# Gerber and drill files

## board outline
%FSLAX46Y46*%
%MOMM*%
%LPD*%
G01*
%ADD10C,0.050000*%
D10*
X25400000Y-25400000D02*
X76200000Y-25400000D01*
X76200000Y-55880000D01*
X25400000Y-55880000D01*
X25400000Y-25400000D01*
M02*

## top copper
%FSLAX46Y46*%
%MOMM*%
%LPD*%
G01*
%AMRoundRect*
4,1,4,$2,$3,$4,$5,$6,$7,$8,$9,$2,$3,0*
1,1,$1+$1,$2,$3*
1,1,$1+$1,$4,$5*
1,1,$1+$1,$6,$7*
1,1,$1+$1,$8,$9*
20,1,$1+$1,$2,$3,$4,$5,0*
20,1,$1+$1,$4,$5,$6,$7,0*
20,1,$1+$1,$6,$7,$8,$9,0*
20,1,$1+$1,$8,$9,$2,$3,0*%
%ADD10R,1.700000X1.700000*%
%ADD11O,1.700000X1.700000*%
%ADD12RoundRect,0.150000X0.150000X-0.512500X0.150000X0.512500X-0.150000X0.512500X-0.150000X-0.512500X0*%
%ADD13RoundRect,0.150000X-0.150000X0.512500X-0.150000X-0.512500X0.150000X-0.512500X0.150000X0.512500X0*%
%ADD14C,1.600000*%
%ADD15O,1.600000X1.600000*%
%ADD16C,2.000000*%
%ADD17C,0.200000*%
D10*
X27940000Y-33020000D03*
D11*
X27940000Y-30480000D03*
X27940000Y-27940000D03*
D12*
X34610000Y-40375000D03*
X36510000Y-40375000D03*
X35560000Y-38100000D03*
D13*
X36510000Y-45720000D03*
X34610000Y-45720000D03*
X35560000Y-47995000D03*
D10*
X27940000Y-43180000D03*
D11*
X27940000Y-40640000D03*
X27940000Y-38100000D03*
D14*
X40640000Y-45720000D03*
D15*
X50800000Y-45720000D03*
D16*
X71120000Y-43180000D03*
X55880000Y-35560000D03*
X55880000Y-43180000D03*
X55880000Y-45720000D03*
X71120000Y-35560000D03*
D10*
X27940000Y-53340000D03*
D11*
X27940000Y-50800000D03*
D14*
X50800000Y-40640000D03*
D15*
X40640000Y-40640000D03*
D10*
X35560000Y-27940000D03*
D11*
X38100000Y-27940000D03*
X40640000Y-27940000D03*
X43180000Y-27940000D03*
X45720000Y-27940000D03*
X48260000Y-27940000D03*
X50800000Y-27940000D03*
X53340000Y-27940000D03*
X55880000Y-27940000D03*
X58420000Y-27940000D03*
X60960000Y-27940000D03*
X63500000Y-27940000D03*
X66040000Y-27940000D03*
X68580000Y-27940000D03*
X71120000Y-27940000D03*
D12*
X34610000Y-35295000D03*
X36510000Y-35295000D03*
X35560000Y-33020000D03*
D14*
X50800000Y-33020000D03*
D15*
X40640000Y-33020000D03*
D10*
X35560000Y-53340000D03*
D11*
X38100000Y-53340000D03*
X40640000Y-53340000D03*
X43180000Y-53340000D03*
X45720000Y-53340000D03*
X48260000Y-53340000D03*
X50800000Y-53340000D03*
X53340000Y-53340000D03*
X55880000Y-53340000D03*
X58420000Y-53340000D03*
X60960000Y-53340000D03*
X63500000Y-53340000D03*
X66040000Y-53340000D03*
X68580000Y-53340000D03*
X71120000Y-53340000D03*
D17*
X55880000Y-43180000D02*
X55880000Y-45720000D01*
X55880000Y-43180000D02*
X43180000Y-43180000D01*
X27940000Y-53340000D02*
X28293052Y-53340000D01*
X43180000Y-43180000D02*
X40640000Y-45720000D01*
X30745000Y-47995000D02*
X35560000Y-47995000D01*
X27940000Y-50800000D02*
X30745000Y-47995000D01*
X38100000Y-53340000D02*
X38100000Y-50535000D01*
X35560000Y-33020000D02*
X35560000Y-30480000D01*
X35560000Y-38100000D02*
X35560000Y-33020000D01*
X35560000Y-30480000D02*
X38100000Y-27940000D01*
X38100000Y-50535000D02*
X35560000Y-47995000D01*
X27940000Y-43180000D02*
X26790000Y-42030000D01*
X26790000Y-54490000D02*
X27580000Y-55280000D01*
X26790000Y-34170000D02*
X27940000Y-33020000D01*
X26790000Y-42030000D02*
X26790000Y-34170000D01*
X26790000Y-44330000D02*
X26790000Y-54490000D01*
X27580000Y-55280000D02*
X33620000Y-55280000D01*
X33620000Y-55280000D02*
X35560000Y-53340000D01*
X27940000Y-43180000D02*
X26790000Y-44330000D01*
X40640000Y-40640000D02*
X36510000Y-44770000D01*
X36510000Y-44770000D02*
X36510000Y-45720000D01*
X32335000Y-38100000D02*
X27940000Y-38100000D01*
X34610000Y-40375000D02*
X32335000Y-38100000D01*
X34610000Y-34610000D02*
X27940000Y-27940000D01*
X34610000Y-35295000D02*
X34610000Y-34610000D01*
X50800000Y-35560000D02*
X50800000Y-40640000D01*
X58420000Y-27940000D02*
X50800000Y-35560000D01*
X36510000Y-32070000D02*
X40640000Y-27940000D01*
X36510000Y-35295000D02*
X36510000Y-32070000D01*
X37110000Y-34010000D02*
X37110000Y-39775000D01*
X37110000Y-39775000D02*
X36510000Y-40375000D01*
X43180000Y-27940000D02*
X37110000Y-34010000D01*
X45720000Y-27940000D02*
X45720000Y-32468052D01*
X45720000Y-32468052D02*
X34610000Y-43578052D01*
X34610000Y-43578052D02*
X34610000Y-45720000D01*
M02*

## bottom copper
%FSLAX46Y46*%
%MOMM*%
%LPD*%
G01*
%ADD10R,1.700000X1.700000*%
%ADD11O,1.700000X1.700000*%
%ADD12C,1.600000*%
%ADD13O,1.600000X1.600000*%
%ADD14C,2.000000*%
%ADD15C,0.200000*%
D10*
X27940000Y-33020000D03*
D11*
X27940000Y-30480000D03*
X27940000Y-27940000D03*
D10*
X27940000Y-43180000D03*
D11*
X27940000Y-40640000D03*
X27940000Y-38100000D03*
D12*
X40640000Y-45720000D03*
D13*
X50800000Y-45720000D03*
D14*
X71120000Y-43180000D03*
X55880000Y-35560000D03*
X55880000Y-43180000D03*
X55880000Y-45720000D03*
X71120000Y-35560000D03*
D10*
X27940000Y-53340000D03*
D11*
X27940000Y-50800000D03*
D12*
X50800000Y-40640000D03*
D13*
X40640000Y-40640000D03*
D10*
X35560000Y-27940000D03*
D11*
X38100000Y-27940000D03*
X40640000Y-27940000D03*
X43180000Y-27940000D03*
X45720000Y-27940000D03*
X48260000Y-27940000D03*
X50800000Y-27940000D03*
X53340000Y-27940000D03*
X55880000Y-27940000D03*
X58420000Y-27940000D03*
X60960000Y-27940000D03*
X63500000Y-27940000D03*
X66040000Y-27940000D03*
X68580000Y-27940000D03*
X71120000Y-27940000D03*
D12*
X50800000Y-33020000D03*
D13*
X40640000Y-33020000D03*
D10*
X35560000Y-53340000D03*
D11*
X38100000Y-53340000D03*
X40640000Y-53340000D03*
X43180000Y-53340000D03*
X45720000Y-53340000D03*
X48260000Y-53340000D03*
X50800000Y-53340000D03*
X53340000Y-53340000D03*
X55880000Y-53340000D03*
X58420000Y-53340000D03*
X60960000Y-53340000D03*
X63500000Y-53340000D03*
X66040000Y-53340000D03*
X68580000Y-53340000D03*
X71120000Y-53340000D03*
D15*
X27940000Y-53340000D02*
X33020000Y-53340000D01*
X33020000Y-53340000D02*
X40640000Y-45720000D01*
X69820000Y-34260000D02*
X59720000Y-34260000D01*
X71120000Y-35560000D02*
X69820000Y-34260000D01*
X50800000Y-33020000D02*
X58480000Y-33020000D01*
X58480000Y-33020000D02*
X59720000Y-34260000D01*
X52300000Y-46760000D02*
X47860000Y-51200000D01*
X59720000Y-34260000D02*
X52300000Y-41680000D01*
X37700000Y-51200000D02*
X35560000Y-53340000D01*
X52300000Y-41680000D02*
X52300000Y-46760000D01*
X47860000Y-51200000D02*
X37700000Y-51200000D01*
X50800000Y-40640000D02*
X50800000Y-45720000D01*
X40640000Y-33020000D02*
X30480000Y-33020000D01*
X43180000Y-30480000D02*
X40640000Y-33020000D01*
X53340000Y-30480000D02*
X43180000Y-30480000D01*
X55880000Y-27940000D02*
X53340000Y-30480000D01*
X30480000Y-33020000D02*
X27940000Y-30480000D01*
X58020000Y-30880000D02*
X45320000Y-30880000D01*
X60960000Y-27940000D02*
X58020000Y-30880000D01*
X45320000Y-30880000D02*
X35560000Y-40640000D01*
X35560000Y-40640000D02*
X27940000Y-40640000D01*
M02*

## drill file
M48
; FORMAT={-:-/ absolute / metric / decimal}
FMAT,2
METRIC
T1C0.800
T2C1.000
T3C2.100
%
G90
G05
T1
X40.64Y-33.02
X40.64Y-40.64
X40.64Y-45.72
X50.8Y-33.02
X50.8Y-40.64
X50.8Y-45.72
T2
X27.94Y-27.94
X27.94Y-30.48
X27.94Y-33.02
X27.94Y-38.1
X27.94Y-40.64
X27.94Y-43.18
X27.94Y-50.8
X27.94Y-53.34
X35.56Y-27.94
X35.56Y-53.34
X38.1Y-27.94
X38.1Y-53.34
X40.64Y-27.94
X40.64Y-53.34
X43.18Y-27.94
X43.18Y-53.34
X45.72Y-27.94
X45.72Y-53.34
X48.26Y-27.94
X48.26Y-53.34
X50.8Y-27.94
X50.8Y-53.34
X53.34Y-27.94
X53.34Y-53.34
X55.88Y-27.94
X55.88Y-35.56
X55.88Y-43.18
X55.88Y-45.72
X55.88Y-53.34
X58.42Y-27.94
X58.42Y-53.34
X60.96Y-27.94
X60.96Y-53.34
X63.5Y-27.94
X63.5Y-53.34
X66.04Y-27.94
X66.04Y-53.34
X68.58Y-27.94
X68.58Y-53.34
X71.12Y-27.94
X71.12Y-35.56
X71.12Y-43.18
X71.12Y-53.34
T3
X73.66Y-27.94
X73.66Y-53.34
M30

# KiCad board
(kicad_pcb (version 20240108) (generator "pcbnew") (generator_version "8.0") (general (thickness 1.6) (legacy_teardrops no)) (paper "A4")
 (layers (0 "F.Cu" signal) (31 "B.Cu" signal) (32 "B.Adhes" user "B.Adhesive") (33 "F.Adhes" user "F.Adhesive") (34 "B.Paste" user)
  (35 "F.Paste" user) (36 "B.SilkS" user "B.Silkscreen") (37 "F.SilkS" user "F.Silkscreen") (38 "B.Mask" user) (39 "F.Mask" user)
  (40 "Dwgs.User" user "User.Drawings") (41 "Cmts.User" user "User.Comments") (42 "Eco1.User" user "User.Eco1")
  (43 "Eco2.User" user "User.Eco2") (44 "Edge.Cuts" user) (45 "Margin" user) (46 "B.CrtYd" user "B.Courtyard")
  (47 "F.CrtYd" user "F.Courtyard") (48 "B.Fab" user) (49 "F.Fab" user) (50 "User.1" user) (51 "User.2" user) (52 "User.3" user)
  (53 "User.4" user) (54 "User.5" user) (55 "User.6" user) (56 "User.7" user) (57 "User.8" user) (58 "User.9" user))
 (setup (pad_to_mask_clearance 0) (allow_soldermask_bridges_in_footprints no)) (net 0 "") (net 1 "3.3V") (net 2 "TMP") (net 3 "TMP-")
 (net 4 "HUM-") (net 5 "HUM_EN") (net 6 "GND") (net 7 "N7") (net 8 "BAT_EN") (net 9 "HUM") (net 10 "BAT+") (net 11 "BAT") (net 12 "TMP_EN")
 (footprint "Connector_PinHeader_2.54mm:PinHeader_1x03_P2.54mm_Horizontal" (layer "F.Cu") (at 27.94 33.02 180)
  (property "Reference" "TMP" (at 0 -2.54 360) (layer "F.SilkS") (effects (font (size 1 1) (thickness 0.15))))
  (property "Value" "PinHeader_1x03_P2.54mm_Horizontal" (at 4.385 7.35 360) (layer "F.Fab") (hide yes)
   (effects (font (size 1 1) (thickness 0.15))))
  (pad "1" thru_hole rect (at 0 0 180) (size 1.7 1.7) (drill 1) (layers "*.Cu" "*.Mask") (remove_unused_layers no) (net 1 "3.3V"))
  (pad "2" thru_hole oval (at 0 2.54 180) (size 1.7 1.7) (drill 1) (layers "*.Cu" "*.Mask") (remove_unused_layers no) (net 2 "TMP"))
  (pad "3" thru_hole oval (at 0 5.08 180) (size 1.7 1.7) (drill 1) (layers "*.Cu" "*.Mask") (remove_unused_layers no) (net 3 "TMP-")))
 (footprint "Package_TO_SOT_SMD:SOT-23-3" (layer "F.Cu") (at 35.56 39.2375 90)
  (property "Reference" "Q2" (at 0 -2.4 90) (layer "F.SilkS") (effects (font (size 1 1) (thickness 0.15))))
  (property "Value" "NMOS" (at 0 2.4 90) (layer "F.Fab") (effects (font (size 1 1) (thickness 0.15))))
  (pad "1" smd roundrect (at -1.1375 -0.95 90) (size 1.325 0.6) (layers "F.Cu" "F.Paste" "F.Mask") (roundrect_rratio 0.25) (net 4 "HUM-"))
  (pad "2" smd roundrect (at -1.1375 0.95 90) (size 1.325 0.6) (layers "F.Cu" "F.Paste" "F.Mask") (roundrect_rratio 0.25) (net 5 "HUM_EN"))
  (pad "3" smd roundrect (at 1.1375 0 90) (size 1.325 0.6) (layers "F.Cu" "F.Paste" "F.Mask") (roundrect_rratio 0.25) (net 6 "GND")))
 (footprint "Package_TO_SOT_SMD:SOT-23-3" (layer "F.Cu") (at 35.56 46.8575 -90)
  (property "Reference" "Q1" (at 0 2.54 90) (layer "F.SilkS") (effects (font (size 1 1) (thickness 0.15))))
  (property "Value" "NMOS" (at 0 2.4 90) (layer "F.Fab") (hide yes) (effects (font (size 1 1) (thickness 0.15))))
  (pad "1" smd roundrect (at -1.1375 -0.95 270) (size 1.325 0.6) (layers "F.Cu" "F.Paste" "F.Mask") (roundrect_rratio 0.25) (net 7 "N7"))
  (pad "2" smd roundrect (at -1.1375 0.95 270) (size 1.325 0.6) (layers "F.Cu" "F.Paste" "F.Mask") (roundrect_rratio 0.25) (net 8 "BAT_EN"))
  (pad "3" smd roundrect (at 1.1375 0 270) (size 1.325 0.6) (layers "F.Cu" "F.Paste" "F.Mask") (roundrect_rratio 0.25) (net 6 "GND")))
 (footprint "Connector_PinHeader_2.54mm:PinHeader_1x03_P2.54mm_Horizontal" (layer "F.Cu") (at 27.94 43.18 180)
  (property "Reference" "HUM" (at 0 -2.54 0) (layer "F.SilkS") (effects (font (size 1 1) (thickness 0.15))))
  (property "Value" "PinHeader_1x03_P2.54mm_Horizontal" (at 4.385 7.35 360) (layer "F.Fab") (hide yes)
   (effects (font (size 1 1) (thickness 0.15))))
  (pad "1" thru_hole rect (at 0 0 180) (size 1.7 1.7) (drill 1) (layers "*.Cu" "*.Mask") (remove_unused_layers no) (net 1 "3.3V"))
  (pad "2" thru_hole oval (at 0 2.54 180) (size 1.7 1.7) (drill 1) (layers "*.Cu" "*.Mask") (remove_unused_layers no) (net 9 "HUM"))
  (pad "3" thru_hole oval (at 0 5.08 180) (size 1.7 1.7) (drill 1) (layers "*.Cu" "*.Mask") (remove_unused_layers no) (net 4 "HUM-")))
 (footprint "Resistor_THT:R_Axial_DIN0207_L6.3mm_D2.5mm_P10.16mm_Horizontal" (layer "F.Cu") (at 40.64 45.72)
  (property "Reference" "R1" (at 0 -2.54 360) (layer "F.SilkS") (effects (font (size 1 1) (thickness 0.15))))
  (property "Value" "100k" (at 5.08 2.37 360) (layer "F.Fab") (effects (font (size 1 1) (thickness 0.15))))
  (pad "1" thru_hole circle (at 0 0) (size 1.6 1.6) (drill 0.8) (layers "*.Cu" "*.Mask") (remove_unused_layers no) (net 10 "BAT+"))
  (pad "2" thru_hole oval (at 10.16 0) (size 1.6 1.6) (drill 0.8) (layers "*.Cu" "*.Mask") (remove_unused_layers no) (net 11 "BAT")))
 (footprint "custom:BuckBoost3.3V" (layer "F.Cu") (at 63.5 40.64 90)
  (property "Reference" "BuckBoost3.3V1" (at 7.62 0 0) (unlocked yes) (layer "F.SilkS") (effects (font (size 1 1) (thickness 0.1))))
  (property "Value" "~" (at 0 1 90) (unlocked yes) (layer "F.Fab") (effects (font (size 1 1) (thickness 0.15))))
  (pad "1" thru_hole circle (at -2.54 7.62 90) (size 2 2) (drill 1) (layers "*.Cu" "*.Mask") (remove_unused_layers no) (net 6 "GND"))
  (pad "1" thru_hole circle (at 5.08 -7.62 90) (size 2 2) (drill 1) (layers "*.Cu" "*.Mask") (remove_unused_layers no) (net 6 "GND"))
  (pad "2" thru_hole circle (at -2.54 -7.62 90) (size 2 2) (drill 1) (layers "*.Cu" "*.Mask") (remove_unused_layers no) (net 10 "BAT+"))
  (pad "3" thru_hole circle (at -5.08 -7.62 90) (size 2 2) (drill 1) (layers "*.Cu" "*.Mask") (remove_unused_layers no) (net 10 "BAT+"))
  (pad "4" thru_hole circle (at 5.08 7.62 90) (size 2 2) (drill 1) (layers "*.Cu" "*.Mask") (remove_unused_layers no) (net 1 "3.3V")))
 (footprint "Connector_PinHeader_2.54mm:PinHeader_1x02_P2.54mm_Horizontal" (layer "F.Cu") (at 27.94 53.34 180)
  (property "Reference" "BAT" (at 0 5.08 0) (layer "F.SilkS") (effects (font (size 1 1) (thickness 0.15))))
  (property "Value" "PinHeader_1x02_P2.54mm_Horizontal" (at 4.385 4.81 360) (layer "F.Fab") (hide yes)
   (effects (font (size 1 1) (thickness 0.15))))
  (pad "1" thru_hole rect (at 0 0 180) (size 1.7 1.7) (drill 1) (layers "*.Cu" "*.Mask") (remove_unused_layers no) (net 10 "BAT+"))
  (pad "2" thru_hole oval (at 0 2.54 180) (size 1.7 1.7) (drill 1) (layers "*.Cu" "*.Mask") (remove_unused_layers no) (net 6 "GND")))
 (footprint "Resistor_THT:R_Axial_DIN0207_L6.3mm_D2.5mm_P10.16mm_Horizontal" (layer "F.Cu") (at 50.8 40.64 180)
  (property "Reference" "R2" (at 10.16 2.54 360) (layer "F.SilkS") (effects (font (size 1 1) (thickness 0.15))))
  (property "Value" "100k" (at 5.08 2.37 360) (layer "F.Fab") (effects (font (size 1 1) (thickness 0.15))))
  (pad "1" thru_hole circle (at 0 0 180) (size 1.6 1.6) (drill 0.8) (layers "*.Cu" "*.Mask") (remove_unused_layers no) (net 11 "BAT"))
  (pad "2" thru_hole oval (at 10.16 0 180) (size 1.6 1.6) (drill 0.8) (layers "*.Cu" "*.Mask") (remove_unused_layers no) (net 7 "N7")))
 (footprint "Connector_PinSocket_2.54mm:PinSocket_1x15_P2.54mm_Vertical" (layer "F.Cu") (at 35.56 27.94 90)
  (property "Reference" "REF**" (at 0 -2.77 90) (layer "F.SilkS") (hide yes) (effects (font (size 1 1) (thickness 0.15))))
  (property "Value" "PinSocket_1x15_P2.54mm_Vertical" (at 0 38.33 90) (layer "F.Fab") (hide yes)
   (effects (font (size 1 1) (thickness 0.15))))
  (pad "1" thru_hole rect (at 0 0 90) (size 1.7 1.7) (drill 1) (layers "*.Cu" "*.Mask") (remove_unused_layers no))
  (pad "2" thru_hole oval (at 0 2.54 90) (size 1.7 1.7) (drill 1) (layers "*.Cu" "*.Mask") (remove_unused_layers no) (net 6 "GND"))
  (pad "3" thru_hole oval (at 0 5.08 90) (size 1.7 1.7) (drill 1) (layers "*.Cu" "*.Mask") (remove_unused_layers no) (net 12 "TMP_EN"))
  (pad "4" thru_hole oval (at 0 7.62 90) (size 1.7 1.7) (drill 1) (layers "*.Cu" "*.Mask") (remove_unused_layers no) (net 5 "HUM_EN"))
  (pad "5" thru_hole oval (at 0 10.16 90) (size 1.7 1.7) (drill 1) (layers "*.Cu" "*.Mask") (remove_unused_layers no) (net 8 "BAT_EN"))
  (pad "6" thru_hole oval (at 0 12.7 90) (size 1.7 1.7) (drill 1) (layers "*.Cu" "*.Mask") (remove_unused_layers no))
  (pad "7" thru_hole oval (at 0 15.24 90) (size 1.7 1.7) (drill 1) (layers "*.Cu" "*.Mask") (remove_unused_layers no))
  (pad "8" thru_hole oval (at 0 17.78 90) (size 1.7 1.7) (drill 1) (layers "*.Cu" "*.Mask") (remove_unused_layers no))
  (pad "9" thru_hole oval (at 0 20.32 90) (size 1.7 1.7) (drill 1) (layers "*.Cu" "*.Mask") (remove_unused_layers no) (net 2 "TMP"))
  (pad "10" thru_hole oval (at 0 22.86 90) (size 1.7 1.7) (drill 1) (layers "*.Cu" "*.Mask") (remove_unused_layers no) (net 11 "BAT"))
  (pad "11" thru_hole oval (at 0 25.4 90) (size 1.7 1.7) (drill 1) (layers "*.Cu" "*.Mask") (remove_unused_layers no) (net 9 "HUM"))
  (pad "12" thru_hole oval (at 0 27.94 90) (size 1.7 1.7) (drill 1) (layers "*.Cu" "*.Mask") (remove_unused_layers no))
  (pad "13" thru_hole oval (at 0 30.48 90) (size 1.7 1.7) (drill 1) (layers "*.Cu" "*.Mask") (remove_unused_layers no))
  (pad "14" thru_hole oval (at 0 33.02 90) (size 1.7 1.7) (drill 1) (layers "*.Cu" "*.Mask") (remove_unused_layers no))
  (pad "15" thru_hole oval (at 0 35.56 90) (size 1.7 1.7) (drill 1) (layers "*.Cu" "*.Mask") (remove_unused_layers no)))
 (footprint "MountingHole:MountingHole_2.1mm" (layer "F.Cu") (at 73.66 53.34)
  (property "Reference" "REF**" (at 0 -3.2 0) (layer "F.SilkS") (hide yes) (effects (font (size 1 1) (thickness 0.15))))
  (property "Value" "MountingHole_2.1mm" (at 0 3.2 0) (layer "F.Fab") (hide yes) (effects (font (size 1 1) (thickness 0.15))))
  (pad "" np_thru_hole circle (at 0 0) (size 2.1 2.1) (drill 2.1) (layers "*.Cu" "*.Mask")))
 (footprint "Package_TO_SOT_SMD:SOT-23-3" (layer "F.Cu") (at 35.56 34.1575 90)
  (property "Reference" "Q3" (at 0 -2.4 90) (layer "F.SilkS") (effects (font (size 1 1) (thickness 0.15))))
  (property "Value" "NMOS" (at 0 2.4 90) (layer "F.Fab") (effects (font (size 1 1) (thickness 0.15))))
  (pad "1" smd roundrect (at -1.1375 -0.95 90) (size 1.325 0.6) (layers "F.Cu" "F.Paste" "F.Mask") (roundrect_rratio 0.25) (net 3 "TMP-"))
  (pad "2" smd roundrect (at -1.1375 0.95 90) (size 1.325 0.6) (layers "F.Cu" "F.Paste" "F.Mask") (roundrect_rratio 0.25) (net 12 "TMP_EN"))
  (pad "3" smd roundrect (at 1.1375 0 90) (size 1.325 0.6) (layers "F.Cu" "F.Paste" "F.Mask") (roundrect_rratio 0.25) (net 6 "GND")))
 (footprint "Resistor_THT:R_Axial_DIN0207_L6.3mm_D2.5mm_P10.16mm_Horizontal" (layer "F.Cu") (at 50.8 33.02 180)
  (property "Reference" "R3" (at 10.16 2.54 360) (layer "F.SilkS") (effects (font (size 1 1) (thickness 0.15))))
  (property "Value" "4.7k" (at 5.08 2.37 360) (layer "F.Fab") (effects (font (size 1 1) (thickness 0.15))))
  (pad "1" thru_hole circle (at 0 0 180) (size 1.6 1.6) (drill 0.8) (layers "*.Cu" "*.Mask") (remove_unused_layers no) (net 1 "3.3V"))
  (pad "2" thru_hole oval (at 10.16 0 180) (size 1.6 1.6) (drill 0.8) (layers "*.Cu" "*.Mask") (remove_unused_layers no) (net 2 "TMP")))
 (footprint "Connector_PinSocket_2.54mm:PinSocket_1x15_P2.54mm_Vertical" (layer "F.Cu") (at 35.56 53.34 90)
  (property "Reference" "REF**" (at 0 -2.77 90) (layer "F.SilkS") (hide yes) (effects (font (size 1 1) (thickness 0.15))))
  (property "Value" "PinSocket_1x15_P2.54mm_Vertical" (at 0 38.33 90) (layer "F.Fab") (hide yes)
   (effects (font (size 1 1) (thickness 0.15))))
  (pad "1" thru_hole rect (at 0 0 90) (size 1.7 1.7) (drill 1) (layers "*.Cu" "*.Mask") (remove_unused_layers no) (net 1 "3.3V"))
  (pad "2" thru_hole oval (at 0 2.54 90) (size 1.7 1.7) (drill 1) (layers "*.Cu" "*.Mask") (remove_unused_layers no) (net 6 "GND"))
  (pad "3" thru_hole oval (at 0 5.08 90) (size 1.7 1.7) (drill 1) (layers "*.Cu" "*.Mask") (remove_unused_layers no))
  (pad "4" thru_hole oval (at 0 7.62 90) (size 1.7 1.7) (drill 1) (layers "*.Cu" "*.Mask") (remove_unused_layers no))
  (pad "5" thru_hole oval (at 0 10.16 90) (size 1.7 1.7) (drill 1) (layers "*.Cu" "*.Mask") (remove_unused_layers no))
  (pad "6" thru_hole oval (at 0 12.7 90) (size 1.7 1.7) (drill 1) (layers "*.Cu" "*.Mask") (remove_unused_layers no))
  (pad "7" thru_hole oval (at 0 15.24 90) (size 1.7 1.7) (drill 1) (layers "*.Cu" "*.Mask") (remove_unused_layers no))
  (pad "8" thru_hole oval (at 0 17.78 90) (size 1.7 1.7) (drill 1) (layers "*.Cu" "*.Mask") (remove_unused_layers no))
  (pad "9" thru_hole oval (at 0 20.32 90) (size 1.7 1.7) (drill 1) (layers "*.Cu" "*.Mask") (remove_unused_layers no))
  (pad "10" thru_hole oval (at 0 22.86 90) (size 1.7 1.7) (drill 1) (layers "*.Cu" "*.Mask") (remove_unused_layers no))
  (pad "11" thru_hole oval (at 0 25.4 90) (size 1.7 1.7) (drill 1) (layers "*.Cu" "*.Mask") (remove_unused_layers no))
  (pad "12" thru_hole oval (at 0 27.94 90) (size 1.7 1.7) (drill 1) (layers "*.Cu" "*.Mask") (remove_unused_layers no))
  (pad "13" thru_hole oval (at 0 30.48 90) (size 1.7 1.7) (drill 1) (layers "*.Cu" "*.Mask") (remove_unused_layers no))
  (pad "14" thru_hole oval (at 0 33.02 90) (size 1.7 1.7) (drill 1) (layers "*.Cu" "*.Mask") (remove_unused_layers no))
  (pad "15" thru_hole oval (at 0 35.56 90) (size 1.7 1.7) (drill 1) (layers "*.Cu" "*.Mask") (remove_unused_layers no)))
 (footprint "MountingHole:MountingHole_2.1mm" (layer "F.Cu") (at 73.66 27.94)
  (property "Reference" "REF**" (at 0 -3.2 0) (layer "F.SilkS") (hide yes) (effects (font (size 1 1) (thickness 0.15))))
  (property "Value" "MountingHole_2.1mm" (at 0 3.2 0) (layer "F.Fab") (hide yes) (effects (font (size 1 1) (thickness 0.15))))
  (pad "" np_thru_hole circle (at 0 0) (size 2.1 2.1) (drill 2.1) (layers "*.Cu" "*.Mask")))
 (gr_rect (start 25.4 25.4) (end 76.2 55.88) (stroke (width 0.05) (type default)) (fill none) (layer "Edge.Cuts"))
 (segment (start 55.88 43.18) (end 55.88 45.72) (width 0.2) (layer "F.Cu") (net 10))
 (segment (start 55.88 43.18) (end 43.18 43.18) (width 0.2) (layer "F.Cu") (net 10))
 (segment (start 27.94 53.34) (end 28.293052 53.34) (width 0.2) (layer "F.Cu") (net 10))
 (segment (start 43.18 43.18) (end 40.64 45.72) (width 0.2) (layer "F.Cu") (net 10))
 (segment (start 27.94 53.34) (end 33.02 53.34) (width 0.2) (layer "B.Cu") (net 10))
 (segment (start 33.02 53.34) (end 40.64 45.72) (width 0.2) (layer "B.Cu") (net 10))
 (segment (start 30.745 47.995) (end 35.56 47.995) (width 0.2) (layer "F.Cu") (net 6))
 (segment (start 27.94 50.8) (end 30.745 47.995) (width 0.2) (layer "F.Cu") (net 6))
 (segment (start 38.1 53.34) (end 38.1 50.535) (width 0.2) (layer "F.Cu") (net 6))
 (segment (start 35.56 33.02) (end 35.56 30.48) (width 0.2) (layer "F.Cu") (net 6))
 (segment (start 35.56 38.1) (end 35.56 33.02) (width 0.2) (layer "F.Cu") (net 6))
 (segment (start 35.56 30.48) (end 38.1 27.94) (width 0.2) (layer "F.Cu") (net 6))
 (segment (start 38.1 50.535) (end 35.56 47.995) (width 0.2) (layer "F.Cu") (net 6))
 (segment (start 27.94 43.18) (end 26.79 42.03) (width 0.2) (layer "F.Cu") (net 1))
 (segment (start 26.79 54.49) (end 27.58 55.28) (width 0.2) (layer "F.Cu") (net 1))
 (segment (start 26.79 34.17) (end 27.94 33.02) (width 0.2) (layer "F.Cu") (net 1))
 (segment (start 26.79 42.03) (end 26.79 34.17) (width 0.2) (layer "F.Cu") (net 1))
 (segment (start 26.79 44.33) (end 26.79 54.49) (width 0.2) (layer "F.Cu") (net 1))
 (segment (start 27.58 55.28) (end 33.62 55.28) (width 0.2) (layer "F.Cu") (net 1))
 (segment (start 33.62 55.28) (end 35.56 53.34) (width 0.2) (layer "F.Cu") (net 1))
 (segment (start 27.94 43.18) (end 26.79 44.33) (width 0.2) (layer "F.Cu") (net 1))
 (segment (start 69.82 34.26) (end 59.72 34.26) (width 0.2) (layer "B.Cu") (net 1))
 (segment (start 71.12 35.56) (end 69.82 34.26) (width 0.2) (layer "B.Cu") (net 1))
 (segment (start 50.8 33.02) (end 58.48 33.02) (width 0.2) (layer "B.Cu") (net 1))
 (segment (start 58.48 33.02) (end 59.72 34.26) (width 0.2) (layer "B.Cu") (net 1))
 (segment (start 52.3 46.76) (end 47.86 51.2) (width 0.2) (layer "B.Cu") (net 1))
 (segment (start 59.72 34.26) (end 52.3 41.68) (width 0.2) (layer "B.Cu") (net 1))
 (segment (start 37.7 51.2) (end 35.56 53.34) (width 0.2) (layer "B.Cu") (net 1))
 (segment (start 52.3 41.68) (end 52.3 46.76) (width 0.2) (layer "B.Cu") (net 1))
 (segment (start 47.86 51.2) (end 37.7 51.2) (width 0.2) (layer "B.Cu") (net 1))
 (segment (start 40.64 40.64) (end 36.51 44.77) (width 0.2) (layer "F.Cu") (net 7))
 (segment (start 36.51 44.77) (end 36.51 45.72) (width 0.2) (layer "F.Cu") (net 7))
 (segment (start 32.335 38.1) (end 27.94 38.1) (width 0.2) (layer "F.Cu") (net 4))
 (segment (start 34.61 40.375) (end 32.335 38.1) (width 0.2) (layer "F.Cu") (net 4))
 (segment (start 34.61 34.61) (end 27.94 27.94) (width 0.2) (layer "F.Cu") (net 3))
 (segment (start 34.61 35.295) (end 34.61 34.61) (width 0.2) (layer "F.Cu") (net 3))
 (segment (start 50.8 35.56) (end 50.8 40.64) (width 0.2) (layer "F.Cu") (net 11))
 (segment (start 58.42 27.94) (end 50.8 35.56) (width 0.2) (layer "F.Cu") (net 11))
 (segment (start 50.8 40.64) (end 50.8 45.72) (width 0.2) (layer "B.Cu") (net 11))
 (segment (start 40.64 33.02) (end 30.48 33.02) (width 0.2) (layer "B.Cu") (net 2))
 (segment (start 43.18 30.48) (end 40.64 33.02) (width 0.2) (layer "B.Cu") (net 2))
 (segment (start 53.34 30.48) (end 43.18 30.48) (width 0.2) (layer "B.Cu") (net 2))
 (segment (start 55.88 27.94) (end 53.34 30.48) (width 0.2) (layer "B.Cu") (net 2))
 (segment (start 30.48 33.02) (end 27.94 30.48) (width 0.2) (layer "B.Cu") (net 2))
 (segment (start 58.02 30.88) (end 45.32 30.88) (width 0.2) (layer "B.Cu") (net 9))
 (segment (start 60.96 27.94) (end 58.02 30.88) (width 0.2) (layer "B.Cu") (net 9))
 (segment (start 45.32 30.88) (end 35.56 40.64) (width 0.2) (layer "B.Cu") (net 9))
 (segment (start 35.56 40.64) (end 27.94 40.64) (width 0.2) (layer "B.Cu") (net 9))
 (segment (start 36.51 32.07) (end 40.64 27.94) (width 0.2) (layer "F.Cu") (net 12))
 (segment (start 36.51 35.295) (end 36.51 32.07) (width 0.2) (layer "F.Cu") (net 12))
 (segment (start 37.11 34.01) (end 37.11 39.775) (width 0.2) (layer "F.Cu") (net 5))
 (segment (start 37.11 39.775) (end 36.51 40.375) (width 0.2) (layer "F.Cu") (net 5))
 (segment (start 43.18 27.94) (end 37.11 34.01) (width 0.2) (layer "F.Cu") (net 5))
 (segment (start 45.72 27.94) (end 45.72 32.468052) (width 0.2) (layer "F.Cu") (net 8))
 (segment (start 45.72 32.468052) (end 34.61 43.578052) (width 0.2) (layer "F.Cu") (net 8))
 (segment (start 34.61 43.578052) (end 34.61 45.72) (width 0.2) (layer "F.Cu") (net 8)))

